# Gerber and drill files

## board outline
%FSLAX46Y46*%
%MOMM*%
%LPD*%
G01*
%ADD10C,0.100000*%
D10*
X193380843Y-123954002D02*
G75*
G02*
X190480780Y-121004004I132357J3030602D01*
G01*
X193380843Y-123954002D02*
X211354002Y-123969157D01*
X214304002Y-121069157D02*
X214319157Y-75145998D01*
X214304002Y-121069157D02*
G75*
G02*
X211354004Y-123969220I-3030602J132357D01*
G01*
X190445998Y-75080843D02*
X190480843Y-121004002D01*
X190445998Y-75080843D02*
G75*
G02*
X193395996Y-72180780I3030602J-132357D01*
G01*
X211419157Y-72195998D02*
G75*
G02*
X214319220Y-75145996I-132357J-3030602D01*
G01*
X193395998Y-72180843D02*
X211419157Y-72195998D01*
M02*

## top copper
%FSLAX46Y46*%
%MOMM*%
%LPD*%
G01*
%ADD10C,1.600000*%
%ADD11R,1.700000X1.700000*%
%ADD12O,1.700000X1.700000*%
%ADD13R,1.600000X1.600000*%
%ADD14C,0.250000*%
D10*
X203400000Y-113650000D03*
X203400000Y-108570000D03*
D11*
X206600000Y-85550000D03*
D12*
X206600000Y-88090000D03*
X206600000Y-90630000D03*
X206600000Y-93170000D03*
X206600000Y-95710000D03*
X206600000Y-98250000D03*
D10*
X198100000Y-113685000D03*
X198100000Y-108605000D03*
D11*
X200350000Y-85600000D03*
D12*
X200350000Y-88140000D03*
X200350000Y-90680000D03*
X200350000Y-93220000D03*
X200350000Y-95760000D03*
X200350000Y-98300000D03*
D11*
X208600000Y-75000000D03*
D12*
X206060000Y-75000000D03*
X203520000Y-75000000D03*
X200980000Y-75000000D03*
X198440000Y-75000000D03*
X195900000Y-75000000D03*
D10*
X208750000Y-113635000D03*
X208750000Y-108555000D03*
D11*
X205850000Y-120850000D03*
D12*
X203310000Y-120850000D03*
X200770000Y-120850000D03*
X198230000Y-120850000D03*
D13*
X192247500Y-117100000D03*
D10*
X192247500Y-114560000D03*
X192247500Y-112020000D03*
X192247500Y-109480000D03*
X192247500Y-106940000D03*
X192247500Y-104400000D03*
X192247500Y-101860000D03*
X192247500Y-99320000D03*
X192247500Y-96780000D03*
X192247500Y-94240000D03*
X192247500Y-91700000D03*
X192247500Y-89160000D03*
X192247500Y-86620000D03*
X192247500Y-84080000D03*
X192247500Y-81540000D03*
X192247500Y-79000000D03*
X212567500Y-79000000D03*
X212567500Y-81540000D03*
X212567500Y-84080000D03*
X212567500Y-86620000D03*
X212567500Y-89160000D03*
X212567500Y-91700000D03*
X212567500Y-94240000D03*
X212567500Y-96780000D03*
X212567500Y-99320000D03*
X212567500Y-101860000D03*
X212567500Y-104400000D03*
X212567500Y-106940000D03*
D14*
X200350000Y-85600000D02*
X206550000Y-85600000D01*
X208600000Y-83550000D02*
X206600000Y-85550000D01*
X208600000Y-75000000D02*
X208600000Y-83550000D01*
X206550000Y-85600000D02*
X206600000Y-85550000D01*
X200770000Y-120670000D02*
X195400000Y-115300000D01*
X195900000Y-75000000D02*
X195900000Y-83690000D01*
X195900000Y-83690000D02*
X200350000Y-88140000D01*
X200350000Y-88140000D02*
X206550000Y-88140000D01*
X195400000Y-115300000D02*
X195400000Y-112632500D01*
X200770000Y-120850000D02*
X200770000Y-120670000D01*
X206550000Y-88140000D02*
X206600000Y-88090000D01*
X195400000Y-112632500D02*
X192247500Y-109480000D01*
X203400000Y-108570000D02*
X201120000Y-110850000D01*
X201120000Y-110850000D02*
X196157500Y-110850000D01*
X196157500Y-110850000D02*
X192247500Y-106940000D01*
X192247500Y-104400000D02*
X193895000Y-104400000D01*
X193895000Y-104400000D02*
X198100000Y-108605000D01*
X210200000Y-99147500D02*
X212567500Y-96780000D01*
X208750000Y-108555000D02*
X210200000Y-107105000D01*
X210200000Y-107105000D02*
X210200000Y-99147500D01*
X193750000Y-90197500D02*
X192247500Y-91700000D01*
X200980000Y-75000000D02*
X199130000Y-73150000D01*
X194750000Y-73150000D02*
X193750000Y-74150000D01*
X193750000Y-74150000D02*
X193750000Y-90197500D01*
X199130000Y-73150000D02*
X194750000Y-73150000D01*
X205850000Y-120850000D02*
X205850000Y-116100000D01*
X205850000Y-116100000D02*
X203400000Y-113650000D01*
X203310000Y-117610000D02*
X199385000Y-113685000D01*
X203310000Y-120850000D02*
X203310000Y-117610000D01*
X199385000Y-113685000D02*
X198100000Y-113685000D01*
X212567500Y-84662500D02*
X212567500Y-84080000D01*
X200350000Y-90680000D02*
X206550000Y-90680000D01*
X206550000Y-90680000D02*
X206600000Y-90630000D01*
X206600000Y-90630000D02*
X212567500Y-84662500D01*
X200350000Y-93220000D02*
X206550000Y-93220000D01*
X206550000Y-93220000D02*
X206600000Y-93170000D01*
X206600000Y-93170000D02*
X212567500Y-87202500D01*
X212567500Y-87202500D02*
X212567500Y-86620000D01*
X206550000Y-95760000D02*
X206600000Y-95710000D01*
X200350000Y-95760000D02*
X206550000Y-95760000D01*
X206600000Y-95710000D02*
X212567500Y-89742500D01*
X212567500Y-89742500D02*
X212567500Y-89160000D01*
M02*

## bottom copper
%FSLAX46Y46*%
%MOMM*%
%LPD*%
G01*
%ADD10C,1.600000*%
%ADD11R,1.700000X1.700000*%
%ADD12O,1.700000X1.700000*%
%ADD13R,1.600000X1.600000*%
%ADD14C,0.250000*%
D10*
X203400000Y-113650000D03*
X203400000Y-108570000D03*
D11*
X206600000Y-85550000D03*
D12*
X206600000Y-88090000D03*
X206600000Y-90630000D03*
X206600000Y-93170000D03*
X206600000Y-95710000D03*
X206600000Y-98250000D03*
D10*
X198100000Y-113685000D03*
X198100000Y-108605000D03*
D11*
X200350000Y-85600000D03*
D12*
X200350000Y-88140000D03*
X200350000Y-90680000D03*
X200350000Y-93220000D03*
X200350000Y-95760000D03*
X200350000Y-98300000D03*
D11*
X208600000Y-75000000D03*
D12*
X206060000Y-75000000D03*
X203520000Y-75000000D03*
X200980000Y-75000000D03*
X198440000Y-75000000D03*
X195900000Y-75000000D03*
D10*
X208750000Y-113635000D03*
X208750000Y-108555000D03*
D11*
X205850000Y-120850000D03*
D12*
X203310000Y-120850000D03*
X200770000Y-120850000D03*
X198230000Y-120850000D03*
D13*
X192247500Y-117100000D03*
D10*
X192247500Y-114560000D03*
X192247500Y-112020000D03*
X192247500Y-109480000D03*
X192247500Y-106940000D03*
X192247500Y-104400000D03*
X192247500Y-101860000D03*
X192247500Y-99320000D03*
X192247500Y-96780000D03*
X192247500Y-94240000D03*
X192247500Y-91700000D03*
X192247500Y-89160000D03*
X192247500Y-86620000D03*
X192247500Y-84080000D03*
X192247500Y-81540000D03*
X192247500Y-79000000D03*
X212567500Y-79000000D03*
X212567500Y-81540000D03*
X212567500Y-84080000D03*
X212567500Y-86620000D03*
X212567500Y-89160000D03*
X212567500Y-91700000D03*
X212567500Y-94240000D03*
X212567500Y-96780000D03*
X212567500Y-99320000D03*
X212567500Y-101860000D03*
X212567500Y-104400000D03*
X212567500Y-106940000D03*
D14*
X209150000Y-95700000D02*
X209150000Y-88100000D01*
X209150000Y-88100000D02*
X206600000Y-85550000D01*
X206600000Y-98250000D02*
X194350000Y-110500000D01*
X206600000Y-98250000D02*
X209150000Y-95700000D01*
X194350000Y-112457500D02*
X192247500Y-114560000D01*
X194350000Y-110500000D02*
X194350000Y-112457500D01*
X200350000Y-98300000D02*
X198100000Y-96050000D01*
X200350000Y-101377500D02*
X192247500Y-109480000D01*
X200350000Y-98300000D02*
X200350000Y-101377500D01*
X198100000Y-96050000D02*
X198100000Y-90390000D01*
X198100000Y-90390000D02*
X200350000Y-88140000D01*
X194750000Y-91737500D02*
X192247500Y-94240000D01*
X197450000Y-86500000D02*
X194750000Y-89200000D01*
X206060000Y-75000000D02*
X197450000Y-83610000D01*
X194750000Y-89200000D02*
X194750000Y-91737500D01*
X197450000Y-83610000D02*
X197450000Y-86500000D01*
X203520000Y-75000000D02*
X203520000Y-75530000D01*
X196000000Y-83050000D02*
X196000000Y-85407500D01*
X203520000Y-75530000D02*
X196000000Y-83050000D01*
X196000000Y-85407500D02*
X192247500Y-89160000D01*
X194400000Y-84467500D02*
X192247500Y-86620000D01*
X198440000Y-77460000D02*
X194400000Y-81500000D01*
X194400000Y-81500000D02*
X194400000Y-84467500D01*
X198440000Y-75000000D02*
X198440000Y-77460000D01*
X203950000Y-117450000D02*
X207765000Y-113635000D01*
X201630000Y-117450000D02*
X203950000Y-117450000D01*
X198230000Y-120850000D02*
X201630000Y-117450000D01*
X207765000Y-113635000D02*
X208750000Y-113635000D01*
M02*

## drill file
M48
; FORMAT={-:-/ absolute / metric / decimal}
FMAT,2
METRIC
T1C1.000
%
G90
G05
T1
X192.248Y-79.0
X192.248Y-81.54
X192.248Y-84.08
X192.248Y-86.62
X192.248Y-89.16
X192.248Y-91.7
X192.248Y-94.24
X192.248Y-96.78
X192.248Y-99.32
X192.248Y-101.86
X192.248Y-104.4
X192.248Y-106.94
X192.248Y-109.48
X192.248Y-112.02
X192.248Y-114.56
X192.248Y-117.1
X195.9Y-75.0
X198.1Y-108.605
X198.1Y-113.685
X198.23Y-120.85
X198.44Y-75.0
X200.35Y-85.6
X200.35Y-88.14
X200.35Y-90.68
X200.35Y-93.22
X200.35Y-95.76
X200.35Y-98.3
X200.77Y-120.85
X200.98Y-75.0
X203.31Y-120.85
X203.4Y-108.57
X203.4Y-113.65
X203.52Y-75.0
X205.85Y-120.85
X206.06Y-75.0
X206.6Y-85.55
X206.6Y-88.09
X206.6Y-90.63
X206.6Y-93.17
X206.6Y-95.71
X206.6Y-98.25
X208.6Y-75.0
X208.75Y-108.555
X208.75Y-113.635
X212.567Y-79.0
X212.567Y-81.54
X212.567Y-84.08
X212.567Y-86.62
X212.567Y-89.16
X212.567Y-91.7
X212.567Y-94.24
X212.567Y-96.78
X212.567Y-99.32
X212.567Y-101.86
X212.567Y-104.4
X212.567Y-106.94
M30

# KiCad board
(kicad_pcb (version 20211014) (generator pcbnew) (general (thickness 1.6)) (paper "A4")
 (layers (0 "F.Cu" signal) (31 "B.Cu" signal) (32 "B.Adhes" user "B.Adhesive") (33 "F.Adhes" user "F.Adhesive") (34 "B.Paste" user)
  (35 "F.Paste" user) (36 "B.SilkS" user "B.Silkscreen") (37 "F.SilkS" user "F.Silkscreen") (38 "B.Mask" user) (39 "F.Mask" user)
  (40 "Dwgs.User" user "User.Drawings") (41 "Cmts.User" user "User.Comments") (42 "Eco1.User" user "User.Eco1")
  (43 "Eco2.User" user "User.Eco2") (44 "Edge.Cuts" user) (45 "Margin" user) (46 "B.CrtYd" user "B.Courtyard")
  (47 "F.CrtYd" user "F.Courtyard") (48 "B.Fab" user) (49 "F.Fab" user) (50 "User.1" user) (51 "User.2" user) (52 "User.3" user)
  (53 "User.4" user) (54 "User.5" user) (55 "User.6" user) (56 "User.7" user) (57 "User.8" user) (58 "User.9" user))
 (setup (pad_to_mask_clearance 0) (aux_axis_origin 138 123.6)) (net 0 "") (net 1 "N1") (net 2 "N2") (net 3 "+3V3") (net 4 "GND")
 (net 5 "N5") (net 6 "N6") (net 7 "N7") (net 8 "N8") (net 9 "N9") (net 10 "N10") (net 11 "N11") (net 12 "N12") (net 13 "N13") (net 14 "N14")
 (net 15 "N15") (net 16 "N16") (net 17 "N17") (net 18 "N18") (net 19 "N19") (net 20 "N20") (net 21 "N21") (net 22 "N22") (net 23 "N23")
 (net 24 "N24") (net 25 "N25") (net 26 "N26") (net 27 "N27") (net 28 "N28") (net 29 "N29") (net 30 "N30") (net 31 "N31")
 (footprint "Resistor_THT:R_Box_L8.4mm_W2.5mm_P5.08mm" (layer "F.Cu") (at 203.4 113.65 90)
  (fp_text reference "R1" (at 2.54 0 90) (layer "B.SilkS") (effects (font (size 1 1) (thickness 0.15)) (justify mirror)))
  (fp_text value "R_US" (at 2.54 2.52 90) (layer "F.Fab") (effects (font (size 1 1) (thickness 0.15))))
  (pad "1" thru_hole circle (at 0 0 90) (size 1.6 1.6) (drill 1) (layers *.Cu *.Mask) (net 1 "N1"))
  (pad "2" thru_hole circle (at 5.08 0 90) (size 1.6 1.6) (drill 1) (layers *.Cu *.Mask) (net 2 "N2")))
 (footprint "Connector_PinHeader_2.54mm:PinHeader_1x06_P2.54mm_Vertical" (layer "F.Cu") (at 206.6 85.55)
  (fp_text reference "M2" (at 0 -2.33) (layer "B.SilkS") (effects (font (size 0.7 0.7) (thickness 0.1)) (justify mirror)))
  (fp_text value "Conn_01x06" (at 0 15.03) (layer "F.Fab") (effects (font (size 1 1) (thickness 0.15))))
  (pad "1" thru_hole rect (at 0 0) (size 1.7 1.7) (drill 1) (layers *.Cu *.Mask) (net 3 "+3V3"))
  (pad "2" thru_hole oval (at 0 2.54) (size 1.7 1.7) (drill 1) (layers *.Cu *.Mask) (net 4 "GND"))
  (pad "3" thru_hole oval (at 0 5.08) (size 1.7 1.7) (drill 1) (layers *.Cu *.Mask) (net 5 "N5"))
  (pad "4" thru_hole oval (at 0 7.62) (size 1.7 1.7) (drill 1) (layers *.Cu *.Mask) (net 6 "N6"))
  (pad "5" thru_hole oval (at 0 10.16) (size 1.7 1.7) (drill 1) (layers *.Cu *.Mask) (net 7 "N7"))
  (pad "6" thru_hole oval (at 0 12.7) (size 1.7 1.7) (drill 1) (layers *.Cu *.Mask) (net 3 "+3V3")))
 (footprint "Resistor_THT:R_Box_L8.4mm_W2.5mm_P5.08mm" (layer "F.Cu") (at 198.1 113.685 90)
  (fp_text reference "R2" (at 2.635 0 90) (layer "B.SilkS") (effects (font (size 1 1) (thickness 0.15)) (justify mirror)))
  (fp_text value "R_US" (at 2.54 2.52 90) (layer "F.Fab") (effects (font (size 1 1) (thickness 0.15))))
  (pad "1" thru_hole circle (at 0 0 90) (size 1.6 1.6) (drill 1) (layers *.Cu *.Mask) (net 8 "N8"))
  (pad "2" thru_hole circle (at 5.08 0 90) (size 1.6 1.6) (drill 1) (layers *.Cu *.Mask) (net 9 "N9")))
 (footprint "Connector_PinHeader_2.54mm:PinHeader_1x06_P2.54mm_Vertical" (layer "F.Cu") (at 200.35 85.6)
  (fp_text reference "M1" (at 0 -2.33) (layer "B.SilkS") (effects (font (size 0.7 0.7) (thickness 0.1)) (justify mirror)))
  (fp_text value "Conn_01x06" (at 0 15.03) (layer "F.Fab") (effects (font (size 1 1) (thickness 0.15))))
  (pad "1" thru_hole rect (at 0 0) (size 1.7 1.7) (drill 1) (layers *.Cu *.Mask) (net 3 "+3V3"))
  (pad "2" thru_hole oval (at 0 2.54) (size 1.7 1.7) (drill 1) (layers *.Cu *.Mask) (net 4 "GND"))
  (pad "3" thru_hole oval (at 0 5.08) (size 1.7 1.7) (drill 1) (layers *.Cu *.Mask) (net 5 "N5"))
  (pad "4" thru_hole oval (at 0 7.62) (size 1.7 1.7) (drill 1) (layers *.Cu *.Mask) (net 6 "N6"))
  (pad "5" thru_hole oval (at 0 10.16) (size 1.7 1.7) (drill 1) (layers *.Cu *.Mask) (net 7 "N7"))
  (pad "6" thru_hole oval (at 0 12.7) (size 1.7 1.7) (drill 1) (layers *.Cu *.Mask) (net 4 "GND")))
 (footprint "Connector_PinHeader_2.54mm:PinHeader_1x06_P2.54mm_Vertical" (layer "F.Cu") (at 208.6 75 -90)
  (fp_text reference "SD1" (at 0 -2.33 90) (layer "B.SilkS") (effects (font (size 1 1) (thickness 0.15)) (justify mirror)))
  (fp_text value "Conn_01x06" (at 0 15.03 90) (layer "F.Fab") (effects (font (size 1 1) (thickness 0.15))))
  (pad "1" thru_hole rect (at 0 0 270) (size 1.7 1.7) (drill 1) (layers *.Cu *.Mask) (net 3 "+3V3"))
  (pad "2" thru_hole oval (at 0 2.54 270) (size 1.7 1.7) (drill 1) (layers *.Cu *.Mask) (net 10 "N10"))
  (pad "3" thru_hole oval (at 0 5.08 270) (size 1.7 1.7) (drill 1) (layers *.Cu *.Mask) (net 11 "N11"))
  (pad "4" thru_hole oval (at 0 7.62 270) (size 1.7 1.7) (drill 1) (layers *.Cu *.Mask) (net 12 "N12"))
  (pad "5" thru_hole oval (at 0 10.16 270) (size 1.7 1.7) (drill 1) (layers *.Cu *.Mask) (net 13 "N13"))
  (pad "6" thru_hole oval (at 0 12.7 270) (size 1.7 1.7) (drill 1) (layers *.Cu *.Mask) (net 4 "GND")))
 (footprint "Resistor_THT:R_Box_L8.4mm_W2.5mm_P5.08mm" (layer "F.Cu") (at 208.75 113.635 90)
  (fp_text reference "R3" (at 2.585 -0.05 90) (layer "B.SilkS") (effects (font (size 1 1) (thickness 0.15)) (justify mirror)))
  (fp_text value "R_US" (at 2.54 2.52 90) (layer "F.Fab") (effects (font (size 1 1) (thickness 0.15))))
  (pad "1" thru_hole circle (at 0 0 90) (size 1.6 1.6) (drill 1) (layers *.Cu *.Mask) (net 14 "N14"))
  (pad "2" thru_hole circle (at 5.08 0 90) (size 1.6 1.6) (drill 1) (layers *.Cu *.Mask) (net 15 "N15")))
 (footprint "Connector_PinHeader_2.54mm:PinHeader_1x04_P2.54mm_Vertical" (layer "F.Cu") (at 205.85 120.85 -90)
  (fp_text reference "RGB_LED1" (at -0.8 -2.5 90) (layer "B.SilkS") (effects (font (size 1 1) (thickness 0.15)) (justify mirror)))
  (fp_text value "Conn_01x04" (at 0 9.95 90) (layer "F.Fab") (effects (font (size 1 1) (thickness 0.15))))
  (pad "1" thru_hole rect (at 0 0 270) (size 1.7 1.7) (drill 1) (layers *.Cu *.Mask) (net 1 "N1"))
  (pad "2" thru_hole oval (at 0 2.54 270) (size 1.7 1.7) (drill 1) (layers *.Cu *.Mask) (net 8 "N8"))
  (pad "3" thru_hole oval (at 0 5.08 270) (size 1.7 1.7) (drill 1) (layers *.Cu *.Mask) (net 4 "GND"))
  (pad "4" thru_hole oval (at 0 7.62 270) (size 1.7 1.7) (drill 1) (layers *.Cu *.Mask) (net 14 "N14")))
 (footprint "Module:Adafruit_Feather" (layer "B.Cu") (at 192.2475 117.1)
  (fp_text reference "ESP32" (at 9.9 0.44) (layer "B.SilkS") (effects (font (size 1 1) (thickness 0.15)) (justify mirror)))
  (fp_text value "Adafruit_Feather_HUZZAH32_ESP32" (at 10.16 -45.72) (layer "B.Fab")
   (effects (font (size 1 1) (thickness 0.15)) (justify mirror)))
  (pad "1" thru_hole rect (at 0 0 180) (size 1.6 1.6) (drill 1) (layers *.Cu *.Mask) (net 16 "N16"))
  (pad "2" thru_hole circle (at 0 -2.54 180) (size 1.6 1.6) (drill 1) (layers *.Cu *.Mask) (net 3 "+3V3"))
  (pad "3" thru_hole circle (at 0 -5.08 180) (size 1.6 1.6) (drill 1) (layers *.Cu *.Mask) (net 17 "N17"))
  (pad "4" thru_hole circle (at 0 -7.62 180) (size 1.6 1.6) (drill 1) (layers *.Cu *.Mask) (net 4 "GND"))
  (pad "5" thru_hole circle (at 0 -10.16 180) (size 1.6 1.6) (drill 1) (layers *.Cu *.Mask) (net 2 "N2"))
  (pad "6" thru_hole circle (at 0 -12.7 180) (size 1.6 1.6) (drill 1) (layers *.Cu *.Mask) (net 9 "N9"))
  (pad "7" thru_hole circle (at 0 -15.24 180) (size 1.6 1.6) (drill 1) (layers *.Cu *.Mask) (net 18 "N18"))
  (pad "8" thru_hole circle (at 0 -17.78 180) (size 1.6 1.6) (drill 1) (layers *.Cu *.Mask) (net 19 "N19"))
  (pad "9" thru_hole circle (at 0 -20.32 180) (size 1.6 1.6) (drill 1) (layers *.Cu *.Mask) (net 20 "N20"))
  (pad "10" thru_hole circle (at 0 -22.86 180) (size 1.6 1.6) (drill 1) (layers *.Cu *.Mask) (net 10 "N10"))
  (pad "11" thru_hole circle (at 0 -25.4 180) (size 1.6 1.6) (drill 1) (layers *.Cu *.Mask) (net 12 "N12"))
  (pad "12" thru_hole circle (at 0 -27.94 180) (size 1.6 1.6) (drill 1) (layers *.Cu *.Mask) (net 11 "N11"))
  (pad "13" thru_hole circle (at 0 -30.48 180) (size 1.6 1.6) (drill 1) (layers *.Cu *.Mask) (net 13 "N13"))
  (pad "14" thru_hole circle (at 0 -33.02 180) (size 1.6 1.6) (drill 1) (layers *.Cu *.Mask) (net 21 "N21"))
  (pad "15" thru_hole circle (at 0 -35.56 180) (size 1.6 1.6) (drill 1) (layers *.Cu *.Mask) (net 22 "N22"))
  (pad "16" thru_hole circle (at 0 -38.1 180) (size 1.6 1.6) (drill 1) (layers *.Cu *.Mask) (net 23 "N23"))
  (pad "17" thru_hole circle (at 20.32 -38.1 180) (size 1.6 1.6) (drill 1) (layers *.Cu *.Mask) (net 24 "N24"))
  (pad "18" thru_hole circle (at 20.32 -35.56 180) (size 1.6 1.6) (drill 1) (layers *.Cu *.Mask) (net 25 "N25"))
  (pad "19" thru_hole circle (at 20.32 -33.02 180) (size 1.6 1.6) (drill 1) (layers *.Cu *.Mask) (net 5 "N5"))
  (pad "20" thru_hole circle (at 20.32 -30.48 180) (size 1.6 1.6) (drill 1) (layers *.Cu *.Mask) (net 6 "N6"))
  (pad "21" thru_hole circle (at 20.32 -27.94 180) (size 1.6 1.6) (drill 1) (layers *.Cu *.Mask) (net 7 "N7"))
  (pad "22" thru_hole circle (at 20.32 -25.4 180) (size 1.6 1.6) (drill 1) (layers *.Cu *.Mask) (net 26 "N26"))
  (pad "23" thru_hole circle (at 20.32 -22.86 180) (size 1.6 1.6) (drill 1) (layers *.Cu *.Mask) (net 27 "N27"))
  (pad "24" thru_hole circle (at 20.32 -20.32 180) (size 1.6 1.6) (drill 1) (layers *.Cu *.Mask) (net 15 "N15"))
  (pad "25" thru_hole circle (at 20.32 -17.78 180) (size 1.6 1.6) (drill 1) (layers *.Cu *.Mask) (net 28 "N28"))
  (pad "26" thru_hole circle (at 20.32 -15.24 180) (size 1.6 1.6) (drill 1) (layers *.Cu *.Mask) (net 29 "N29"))
  (pad "27" thru_hole circle (at 20.32 -12.7 180) (size 1.6 1.6) (drill 1) (layers *.Cu *.Mask) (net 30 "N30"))
  (pad "28" thru_hole circle (at 20.32 -10.16 180) (size 1.6 1.6) (drill 1) (layers *.Cu *.Mask) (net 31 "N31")))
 (gr_arc (start 193.380843 123.954002) (mid 191.35 123.05) (end 190.480843 121.004002) (layer "Edge.Cuts") (width 0.1))
 (gr_line (start 193.380843 123.954002) (end 211.354002 123.969157) (layer "Edge.Cuts") (width 0.1))
 (gr_line (start 214.304002 121.069157) (end 214.319157 75.145998) (layer "Edge.Cuts") (width 0.1))
 (gr_arc (start 214.304002 121.069157) (mid 213.4 123.1) (end 211.354002 123.969157) (layer "Edge.Cuts") (width 0.1))
 (gr_line (start 190.445998 75.080843) (end 190.480843 121.004002) (layer "Edge.Cuts") (width 0.1))
 (gr_arc (start 190.445998 75.080843) (mid 191.35 73.05) (end 193.395998 72.180843) (layer "Edge.Cuts") (width 0.1))
 (gr_arc (start 211.419157 72.195998) (mid 213.45 73.1) (end 214.319157 75.145998) (layer "Edge.Cuts") (width 0.1))
 (gr_line (start 193.395998 72.180843) (end 211.419157 72.195998) (layer "Edge.Cuts") (width 0.1))
 (segment (start 200.35 85.6) (end 206.55 85.6) (width 0.25) (layer "F.Cu") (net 3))
 (segment (start 208.6 83.55) (end 206.6 85.55) (width 0.25) (layer "F.Cu") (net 3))
 (segment (start 208.6 75) (end 208.6 83.55) (width 0.25) (layer "F.Cu") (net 3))
 (segment (start 206.55 85.6) (end 206.6 85.55) (width 0.25) (layer "F.Cu") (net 3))
 (segment (start 209.15 95.7) (end 209.15 88.1) (width 0.25) (layer "B.Cu") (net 3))
 (segment (start 209.15 88.1) (end 206.6 85.55) (width 0.25) (layer "B.Cu") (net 3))
 (segment (start 206.6 98.25) (end 194.35 110.5) (width 0.25) (layer "B.Cu") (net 3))
 (segment (start 206.6 98.25) (end 209.15 95.7) (width 0.25) (layer "B.Cu") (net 3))
 (segment (start 194.35 112.4575) (end 192.2475 114.56) (width 0.25) (layer "B.Cu") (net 3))
 (segment (start 194.35 110.5) (end 194.35 112.4575) (width 0.25) (layer "B.Cu") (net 3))
 (segment (start 200.77 120.67) (end 195.4 115.3) (width 0.25) (layer "F.Cu") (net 4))
 (segment (start 195.9 75) (end 195.9 83.69) (width 0.25) (layer "F.Cu") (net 4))
 (segment (start 195.9 83.69) (end 200.35 88.14) (width 0.25) (layer "F.Cu") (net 4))
 (segment (start 200.35 88.14) (end 206.55 88.14) (width 0.25) (layer "F.Cu") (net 4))
 (segment (start 195.4 115.3) (end 195.4 112.6325) (width 0.25) (layer "F.Cu") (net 4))
 (segment (start 200.77 120.85) (end 200.77 120.67) (width 0.25) (layer "F.Cu") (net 4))
 (segment (start 206.55 88.14) (end 206.6 88.09) (width 0.25) (layer "F.Cu") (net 4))
 (segment (start 195.4 112.6325) (end 192.2475 109.48) (width 0.25) (layer "F.Cu") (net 4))
 (segment (start 200.35 98.3) (end 198.1 96.05) (width 0.25) (layer "B.Cu") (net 4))
 (segment (start 200.35 101.3775) (end 192.2475 109.48) (width 0.25) (layer "B.Cu") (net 4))
 (segment (start 200.35 98.3) (end 200.35 101.3775) (width 0.25) (layer "B.Cu") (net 4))
 (segment (start 198.1 96.05) (end 198.1 90.39) (width 0.25) (layer "B.Cu") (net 4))
 (segment (start 198.1 90.39) (end 200.35 88.14) (width 0.25) (layer "B.Cu") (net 4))
 (segment (start 203.4 108.57) (end 201.12 110.85) (width 0.25) (layer "F.Cu") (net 2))
 (segment (start 201.12 110.85) (end 196.1575 110.85) (width 0.25) (layer "F.Cu") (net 2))
 (segment (start 196.1575 110.85) (end 192.2475 106.94) (width 0.25) (layer "F.Cu") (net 2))
 (segment (start 192.2475 104.4) (end 193.895 104.4) (width 0.25) (layer "F.Cu") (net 9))
 (segment (start 193.895 104.4) (end 198.1 108.605) (width 0.25) (layer "F.Cu") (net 9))
 (segment (start 210.2 99.1475) (end 212.5675 96.78) (width 0.25) (layer "F.Cu") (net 15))
 (segment (start 208.75 108.555) (end 210.2 107.105) (width 0.25) (layer "F.Cu") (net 15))
 (segment (start 210.2 107.105) (end 210.2 99.1475) (width 0.25) (layer "F.Cu") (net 15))
 (segment (start 194.75 91.7375) (end 192.2475 94.24) (width 0.25) (layer "B.Cu") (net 10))
 (segment (start 197.45 86.5) (end 194.75 89.2) (width 0.25) (layer "B.Cu") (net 10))
 (segment (start 206.06 75) (end 197.45 83.61) (width 0.25) (layer "B.Cu") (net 10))
 (segment (start 194.75 89.2) (end 194.75 91.7375) (width 0.25) (layer "B.Cu") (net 10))
 (segment (start 197.45 83.61) (end 197.45 86.5) (width 0.25) (layer "B.Cu") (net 10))
 (segment (start 193.75 90.1975) (end 192.2475 91.7) (width 0.25) (layer "F.Cu") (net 12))
 (segment (start 200.98 75) (end 199.13 73.15) (width 0.25) (layer "F.Cu") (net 12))
 (segment (start 194.75 73.15) (end 193.75 74.15) (width 0.25) (layer "F.Cu") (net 12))
 (segment (start 193.75 74.15) (end 193.75 90.1975) (width 0.25) (layer "F.Cu") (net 12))
 (segment (start 199.13 73.15) (end 194.75 73.15) (width 0.25) (layer "F.Cu") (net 12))
 (segment (start 203.52 75) (end 203.52 75.53) (width 0.25) (layer "B.Cu") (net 11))
 (segment (start 196 83.05) (end 196 85.4075) (width 0.25) (layer "B.Cu") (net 11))
 (segment (start 203.52 75.53) (end 196 83.05) (width 0.25) (layer "B.Cu") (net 11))
 (segment (start 196 85.4075) (end 192.2475 89.16) (width 0.25) (layer "B.Cu") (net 11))
 (segment (start 194.4 84.4675) (end 192.2475 86.62) (width 0.25) (layer "B.Cu") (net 13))
 (segment (start 198.44 77.46) (end 194.4 81.5) (width 0.25) (layer "B.Cu") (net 13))
 (segment (start 194.4 81.5) (end 194.4 84.4675) (width 0.25) (layer "B.Cu") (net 13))
 (segment (start 198.44 75) (end 198.44 77.46) (width 0.25) (layer "B.Cu") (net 13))
 (segment (start 205.85 120.85) (end 205.85 116.1) (width 0.25) (layer "F.Cu") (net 1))
 (segment (start 205.85 116.1) (end 203.4 113.65) (width 0.25) (layer "F.Cu") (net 1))
 (segment (start 203.31 117.61) (end 199.385 113.685) (width 0.25) (layer "F.Cu") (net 8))
 (segment (start 203.31 120.85) (end 203.31 117.61) (width 0.25) (layer "F.Cu") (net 8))
 (segment (start 199.385 113.685) (end 198.1 113.685) (width 0.25) (layer "F.Cu") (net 8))
 (segment (start 203.95 117.45) (end 207.765 113.635) (width 0.25) (layer "B.Cu") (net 14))
 (segment (start 201.63 117.45) (end 203.95 117.45) (width 0.25) (layer "B.Cu") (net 14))
 (segment (start 198.23 120.85) (end 201.63 117.45) (width 0.25) (layer "B.Cu") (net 14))
 (segment (start 207.765 113.635) (end 208.75 113.635) (width 0.25) (layer "B.Cu") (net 14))
 (segment (start 212.5675 84.6625) (end 212.5675 84.08) (width 0.25) (layer "F.Cu") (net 5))
 (segment (start 200.35 90.68) (end 206.55 90.68) (width 0.25) (layer "F.Cu") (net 5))
 (segment (start 206.55 90.68) (end 206.6 90.63) (width 0.25) (layer "F.Cu") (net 5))
 (segment (start 206.6 90.63) (end 212.5675 84.6625) (width 0.25) (layer "F.Cu") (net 5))
 (segment (start 200.35 93.22) (end 206.55 93.22) (width 0.25) (layer "F.Cu") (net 6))
 (segment (start 206.55 93.22) (end 206.6 93.17) (width 0.25) (layer "F.Cu") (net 6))
 (segment (start 206.6 93.17) (end 212.5675 87.2025) (width 0.25) (layer "F.Cu") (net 6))
 (segment (start 212.5675 87.2025) (end 212.5675 86.62) (width 0.25) (layer "F.Cu") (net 6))
 (segment (start 206.55 95.76) (end 206.6 95.71) (width 0.25) (layer "F.Cu") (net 7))
 (segment (start 200.35 95.76) (end 206.55 95.76) (width 0.25) (layer "F.Cu") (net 7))
 (segment (start 206.6 95.71) (end 212.5675 89.7425) (width 0.25) (layer "F.Cu") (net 7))
 (segment (start 212.5675 89.7425) (end 212.5675 89.16) (width 0.25) (layer "F.Cu") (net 7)))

